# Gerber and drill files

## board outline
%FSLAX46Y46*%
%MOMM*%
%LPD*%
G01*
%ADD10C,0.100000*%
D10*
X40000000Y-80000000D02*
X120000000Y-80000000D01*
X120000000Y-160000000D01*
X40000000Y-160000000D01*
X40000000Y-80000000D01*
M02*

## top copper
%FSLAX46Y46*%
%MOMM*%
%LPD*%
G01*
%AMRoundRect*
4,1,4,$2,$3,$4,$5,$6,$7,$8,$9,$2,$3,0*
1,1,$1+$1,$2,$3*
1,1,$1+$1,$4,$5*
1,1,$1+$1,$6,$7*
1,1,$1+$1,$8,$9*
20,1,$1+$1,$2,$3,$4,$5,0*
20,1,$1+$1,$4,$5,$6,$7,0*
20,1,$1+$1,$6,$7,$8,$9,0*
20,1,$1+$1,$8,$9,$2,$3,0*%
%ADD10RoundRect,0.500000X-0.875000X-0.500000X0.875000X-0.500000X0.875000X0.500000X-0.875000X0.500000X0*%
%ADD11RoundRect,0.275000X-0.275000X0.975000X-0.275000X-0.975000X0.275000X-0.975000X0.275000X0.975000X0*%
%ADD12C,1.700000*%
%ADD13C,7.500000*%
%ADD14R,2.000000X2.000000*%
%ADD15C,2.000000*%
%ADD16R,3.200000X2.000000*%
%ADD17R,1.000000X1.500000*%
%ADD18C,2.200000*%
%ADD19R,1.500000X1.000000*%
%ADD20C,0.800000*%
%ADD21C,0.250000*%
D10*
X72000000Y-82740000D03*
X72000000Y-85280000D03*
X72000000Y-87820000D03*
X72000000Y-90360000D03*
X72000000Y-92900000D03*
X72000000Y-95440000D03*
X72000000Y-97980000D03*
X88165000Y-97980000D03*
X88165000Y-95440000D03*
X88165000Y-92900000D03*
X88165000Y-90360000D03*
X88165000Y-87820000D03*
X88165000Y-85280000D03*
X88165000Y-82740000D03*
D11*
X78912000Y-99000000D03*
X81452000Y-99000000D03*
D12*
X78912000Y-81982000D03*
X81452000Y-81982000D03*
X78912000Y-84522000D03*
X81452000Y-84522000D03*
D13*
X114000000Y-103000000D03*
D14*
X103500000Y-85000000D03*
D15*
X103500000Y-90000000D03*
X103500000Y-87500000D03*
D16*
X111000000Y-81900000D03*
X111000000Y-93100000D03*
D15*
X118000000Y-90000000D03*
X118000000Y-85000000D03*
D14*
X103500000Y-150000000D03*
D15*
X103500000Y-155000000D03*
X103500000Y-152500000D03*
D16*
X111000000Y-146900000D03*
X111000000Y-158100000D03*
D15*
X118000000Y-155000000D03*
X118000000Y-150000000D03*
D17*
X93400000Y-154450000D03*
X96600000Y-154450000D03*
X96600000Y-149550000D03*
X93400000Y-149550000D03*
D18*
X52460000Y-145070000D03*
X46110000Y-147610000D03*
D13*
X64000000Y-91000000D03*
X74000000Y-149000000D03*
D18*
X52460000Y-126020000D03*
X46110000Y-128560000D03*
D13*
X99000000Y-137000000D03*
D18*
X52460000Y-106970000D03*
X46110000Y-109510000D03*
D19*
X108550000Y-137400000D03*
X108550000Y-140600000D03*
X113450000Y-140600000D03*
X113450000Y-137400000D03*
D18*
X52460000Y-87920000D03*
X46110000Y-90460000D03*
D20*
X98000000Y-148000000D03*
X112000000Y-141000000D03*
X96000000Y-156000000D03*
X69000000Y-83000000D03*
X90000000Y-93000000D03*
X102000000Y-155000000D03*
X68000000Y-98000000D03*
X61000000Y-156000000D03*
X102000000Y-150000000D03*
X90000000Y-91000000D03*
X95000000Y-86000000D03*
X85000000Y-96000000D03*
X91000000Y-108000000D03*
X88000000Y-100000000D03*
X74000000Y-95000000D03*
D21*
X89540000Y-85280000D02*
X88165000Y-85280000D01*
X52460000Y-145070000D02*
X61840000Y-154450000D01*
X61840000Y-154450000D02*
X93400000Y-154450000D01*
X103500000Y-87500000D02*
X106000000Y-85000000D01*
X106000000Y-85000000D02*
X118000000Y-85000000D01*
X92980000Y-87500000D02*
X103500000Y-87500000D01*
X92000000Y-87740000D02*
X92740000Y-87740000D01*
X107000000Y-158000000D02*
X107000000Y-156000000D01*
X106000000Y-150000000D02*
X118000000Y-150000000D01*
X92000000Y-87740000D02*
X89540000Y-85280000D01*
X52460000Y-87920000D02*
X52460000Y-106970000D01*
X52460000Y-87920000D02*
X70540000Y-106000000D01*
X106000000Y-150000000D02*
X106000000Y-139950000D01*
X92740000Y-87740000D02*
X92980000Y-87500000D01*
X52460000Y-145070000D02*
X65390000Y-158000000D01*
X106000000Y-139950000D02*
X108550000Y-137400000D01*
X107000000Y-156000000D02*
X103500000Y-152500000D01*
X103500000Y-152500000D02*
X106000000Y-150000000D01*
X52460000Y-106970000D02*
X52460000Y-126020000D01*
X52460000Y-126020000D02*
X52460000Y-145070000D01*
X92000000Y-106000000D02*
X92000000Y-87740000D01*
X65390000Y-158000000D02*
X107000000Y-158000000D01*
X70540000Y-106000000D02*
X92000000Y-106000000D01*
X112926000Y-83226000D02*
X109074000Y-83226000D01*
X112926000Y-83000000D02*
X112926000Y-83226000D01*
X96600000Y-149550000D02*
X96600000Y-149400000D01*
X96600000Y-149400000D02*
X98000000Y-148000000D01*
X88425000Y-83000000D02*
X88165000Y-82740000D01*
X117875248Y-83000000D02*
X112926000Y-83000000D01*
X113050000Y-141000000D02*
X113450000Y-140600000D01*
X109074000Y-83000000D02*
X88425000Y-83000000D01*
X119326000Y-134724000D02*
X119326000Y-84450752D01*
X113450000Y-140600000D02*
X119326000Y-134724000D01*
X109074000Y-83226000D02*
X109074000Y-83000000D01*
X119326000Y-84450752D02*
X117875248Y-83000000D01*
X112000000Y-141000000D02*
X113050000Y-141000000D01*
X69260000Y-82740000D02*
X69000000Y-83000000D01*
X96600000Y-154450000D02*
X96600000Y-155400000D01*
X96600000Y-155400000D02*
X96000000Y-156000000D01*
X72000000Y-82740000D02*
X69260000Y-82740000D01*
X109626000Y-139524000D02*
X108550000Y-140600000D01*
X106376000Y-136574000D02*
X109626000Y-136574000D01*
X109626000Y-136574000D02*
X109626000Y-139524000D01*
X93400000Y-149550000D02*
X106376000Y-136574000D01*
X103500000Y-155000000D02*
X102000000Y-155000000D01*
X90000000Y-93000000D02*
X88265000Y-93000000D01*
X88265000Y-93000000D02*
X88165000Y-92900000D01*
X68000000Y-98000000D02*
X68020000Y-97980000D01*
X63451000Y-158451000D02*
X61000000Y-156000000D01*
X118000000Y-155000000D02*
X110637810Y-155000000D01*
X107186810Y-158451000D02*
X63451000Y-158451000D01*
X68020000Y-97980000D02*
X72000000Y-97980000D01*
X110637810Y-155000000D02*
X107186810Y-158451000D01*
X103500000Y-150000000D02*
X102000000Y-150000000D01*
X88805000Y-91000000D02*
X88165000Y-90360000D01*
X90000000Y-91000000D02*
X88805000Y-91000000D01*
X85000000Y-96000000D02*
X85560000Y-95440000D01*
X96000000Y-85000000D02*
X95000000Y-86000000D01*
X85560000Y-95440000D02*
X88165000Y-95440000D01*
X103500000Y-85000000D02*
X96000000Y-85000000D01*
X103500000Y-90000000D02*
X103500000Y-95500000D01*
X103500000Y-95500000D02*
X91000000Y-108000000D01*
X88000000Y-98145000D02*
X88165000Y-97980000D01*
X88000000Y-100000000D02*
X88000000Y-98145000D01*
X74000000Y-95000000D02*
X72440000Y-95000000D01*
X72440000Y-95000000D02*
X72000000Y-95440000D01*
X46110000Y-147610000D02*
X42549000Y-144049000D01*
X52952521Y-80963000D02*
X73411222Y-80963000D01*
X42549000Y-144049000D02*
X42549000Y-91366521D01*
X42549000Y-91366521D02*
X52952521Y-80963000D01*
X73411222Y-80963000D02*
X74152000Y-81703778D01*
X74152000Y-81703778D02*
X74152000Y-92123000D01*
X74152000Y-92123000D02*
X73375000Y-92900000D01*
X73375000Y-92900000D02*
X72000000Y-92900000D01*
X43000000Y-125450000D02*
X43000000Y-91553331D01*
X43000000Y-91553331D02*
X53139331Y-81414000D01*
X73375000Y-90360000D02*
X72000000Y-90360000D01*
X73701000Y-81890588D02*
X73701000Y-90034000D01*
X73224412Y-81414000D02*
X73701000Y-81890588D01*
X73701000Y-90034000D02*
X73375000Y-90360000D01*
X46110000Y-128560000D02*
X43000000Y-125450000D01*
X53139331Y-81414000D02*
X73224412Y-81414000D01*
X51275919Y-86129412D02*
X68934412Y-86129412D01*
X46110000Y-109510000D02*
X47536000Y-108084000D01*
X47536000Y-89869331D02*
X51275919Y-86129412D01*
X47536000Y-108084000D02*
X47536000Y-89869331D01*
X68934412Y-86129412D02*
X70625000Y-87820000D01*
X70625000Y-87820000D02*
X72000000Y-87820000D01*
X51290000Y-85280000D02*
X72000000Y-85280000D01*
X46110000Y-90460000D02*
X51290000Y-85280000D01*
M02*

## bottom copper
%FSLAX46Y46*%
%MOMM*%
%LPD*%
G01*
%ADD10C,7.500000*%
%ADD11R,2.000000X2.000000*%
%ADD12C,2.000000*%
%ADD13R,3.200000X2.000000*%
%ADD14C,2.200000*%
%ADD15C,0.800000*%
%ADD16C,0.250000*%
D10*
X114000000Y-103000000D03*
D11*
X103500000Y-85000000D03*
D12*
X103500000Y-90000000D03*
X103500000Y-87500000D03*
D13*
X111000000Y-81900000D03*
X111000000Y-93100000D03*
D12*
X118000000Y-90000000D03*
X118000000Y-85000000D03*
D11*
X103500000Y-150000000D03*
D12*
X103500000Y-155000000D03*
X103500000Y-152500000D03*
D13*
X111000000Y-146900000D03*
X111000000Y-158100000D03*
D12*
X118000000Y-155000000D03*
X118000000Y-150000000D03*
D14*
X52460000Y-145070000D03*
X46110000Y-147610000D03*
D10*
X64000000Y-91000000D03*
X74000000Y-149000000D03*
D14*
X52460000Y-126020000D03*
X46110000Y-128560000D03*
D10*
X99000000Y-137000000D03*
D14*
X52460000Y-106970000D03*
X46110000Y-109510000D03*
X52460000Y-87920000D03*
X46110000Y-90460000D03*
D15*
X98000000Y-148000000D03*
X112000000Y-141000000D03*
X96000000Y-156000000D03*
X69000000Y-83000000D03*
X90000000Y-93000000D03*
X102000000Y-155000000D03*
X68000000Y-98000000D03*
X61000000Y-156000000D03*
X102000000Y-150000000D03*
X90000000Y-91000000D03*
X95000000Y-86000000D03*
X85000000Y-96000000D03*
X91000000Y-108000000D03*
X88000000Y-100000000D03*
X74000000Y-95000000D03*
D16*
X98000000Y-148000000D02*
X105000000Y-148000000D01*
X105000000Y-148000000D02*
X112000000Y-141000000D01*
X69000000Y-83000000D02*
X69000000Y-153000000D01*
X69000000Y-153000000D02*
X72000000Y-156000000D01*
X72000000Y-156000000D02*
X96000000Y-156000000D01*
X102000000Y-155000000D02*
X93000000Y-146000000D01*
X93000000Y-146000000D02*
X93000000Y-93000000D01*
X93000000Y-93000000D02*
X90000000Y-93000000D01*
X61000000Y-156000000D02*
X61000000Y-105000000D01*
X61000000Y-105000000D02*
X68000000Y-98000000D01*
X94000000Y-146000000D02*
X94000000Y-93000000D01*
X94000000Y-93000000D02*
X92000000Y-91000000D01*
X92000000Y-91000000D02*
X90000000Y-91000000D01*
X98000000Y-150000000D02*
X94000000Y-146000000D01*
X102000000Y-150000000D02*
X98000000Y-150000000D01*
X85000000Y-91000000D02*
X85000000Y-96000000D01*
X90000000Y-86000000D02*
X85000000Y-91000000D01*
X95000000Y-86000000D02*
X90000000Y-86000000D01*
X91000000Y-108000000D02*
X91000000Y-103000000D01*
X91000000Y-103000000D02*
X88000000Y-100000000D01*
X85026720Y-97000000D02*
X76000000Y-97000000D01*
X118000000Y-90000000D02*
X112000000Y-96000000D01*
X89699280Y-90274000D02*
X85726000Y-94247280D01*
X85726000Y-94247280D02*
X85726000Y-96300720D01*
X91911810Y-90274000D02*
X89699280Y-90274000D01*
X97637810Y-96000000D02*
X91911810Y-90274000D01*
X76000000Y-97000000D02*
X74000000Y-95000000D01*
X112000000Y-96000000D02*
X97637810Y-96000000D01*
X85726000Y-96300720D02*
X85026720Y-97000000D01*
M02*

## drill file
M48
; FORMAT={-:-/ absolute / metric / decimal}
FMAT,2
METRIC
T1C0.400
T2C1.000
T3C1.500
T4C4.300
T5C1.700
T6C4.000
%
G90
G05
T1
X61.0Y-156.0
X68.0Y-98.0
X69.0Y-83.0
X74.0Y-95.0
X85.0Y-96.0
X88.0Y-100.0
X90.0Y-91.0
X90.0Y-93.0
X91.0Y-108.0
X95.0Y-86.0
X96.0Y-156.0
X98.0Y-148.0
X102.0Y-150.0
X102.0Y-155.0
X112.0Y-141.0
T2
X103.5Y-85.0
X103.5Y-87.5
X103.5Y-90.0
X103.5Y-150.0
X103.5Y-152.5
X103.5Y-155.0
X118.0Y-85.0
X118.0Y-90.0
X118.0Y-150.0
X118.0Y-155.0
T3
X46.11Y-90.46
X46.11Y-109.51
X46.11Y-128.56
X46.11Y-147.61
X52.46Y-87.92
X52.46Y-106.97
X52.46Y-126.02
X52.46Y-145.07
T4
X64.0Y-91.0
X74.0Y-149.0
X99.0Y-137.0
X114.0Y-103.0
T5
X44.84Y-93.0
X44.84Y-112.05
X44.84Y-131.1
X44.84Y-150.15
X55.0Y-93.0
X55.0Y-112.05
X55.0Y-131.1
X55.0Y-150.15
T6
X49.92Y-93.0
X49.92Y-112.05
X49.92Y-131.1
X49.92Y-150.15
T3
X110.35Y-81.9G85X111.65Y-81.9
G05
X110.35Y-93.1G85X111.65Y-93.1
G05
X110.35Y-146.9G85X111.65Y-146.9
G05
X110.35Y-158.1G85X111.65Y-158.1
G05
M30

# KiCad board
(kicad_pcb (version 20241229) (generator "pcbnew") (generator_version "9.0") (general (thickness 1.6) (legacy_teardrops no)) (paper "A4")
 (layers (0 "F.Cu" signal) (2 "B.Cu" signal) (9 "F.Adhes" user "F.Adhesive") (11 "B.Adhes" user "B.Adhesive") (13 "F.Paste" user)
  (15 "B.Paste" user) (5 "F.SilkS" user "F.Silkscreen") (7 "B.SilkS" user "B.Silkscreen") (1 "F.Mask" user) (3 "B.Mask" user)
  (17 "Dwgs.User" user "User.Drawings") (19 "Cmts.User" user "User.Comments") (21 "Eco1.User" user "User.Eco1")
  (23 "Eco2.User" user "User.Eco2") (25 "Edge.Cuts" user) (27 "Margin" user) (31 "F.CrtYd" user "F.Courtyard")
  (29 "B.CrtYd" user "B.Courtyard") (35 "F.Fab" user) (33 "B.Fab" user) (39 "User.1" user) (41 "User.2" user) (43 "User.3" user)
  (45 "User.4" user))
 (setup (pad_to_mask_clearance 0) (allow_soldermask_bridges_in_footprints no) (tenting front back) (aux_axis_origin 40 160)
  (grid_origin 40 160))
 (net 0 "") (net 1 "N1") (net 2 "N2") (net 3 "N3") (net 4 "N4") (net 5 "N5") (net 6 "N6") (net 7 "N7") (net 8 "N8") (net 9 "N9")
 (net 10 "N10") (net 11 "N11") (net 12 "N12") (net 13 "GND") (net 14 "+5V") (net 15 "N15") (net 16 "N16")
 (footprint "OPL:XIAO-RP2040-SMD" (layer "F.Cu") (at 80 90.36)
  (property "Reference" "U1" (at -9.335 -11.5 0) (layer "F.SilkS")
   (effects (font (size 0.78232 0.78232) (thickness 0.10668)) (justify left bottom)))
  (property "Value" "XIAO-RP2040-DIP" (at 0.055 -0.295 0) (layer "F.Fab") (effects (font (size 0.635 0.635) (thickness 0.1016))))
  (pad "1" smd roundrect (at -8 -7.62) (size 2.75 2) (layers "F.Cu" "F.Mask" "F.Paste") (roundrect_rratio 0.25) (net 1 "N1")
   (solder_mask_margin 0.0508) (thermal_bridge_angle 45))
  (pad "2" smd roundrect (at -8 -5.08) (size 2.75 2) (layers "F.Cu" "F.Mask" "F.Paste") (roundrect_rratio 0.25) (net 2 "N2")
   (solder_mask_margin 0.0508) (thermal_bridge_angle 45))
  (pad "3" smd roundrect (at -8 -2.54) (size 2.75 2) (layers "F.Cu" "F.Mask" "F.Paste") (roundrect_rratio 0.25) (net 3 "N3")
   (solder_mask_margin 0.0508) (thermal_bridge_angle 45))
  (pad "4" smd roundrect (at -8 0) (size 2.75 2) (layers "F.Cu" "F.Mask" "F.Paste") (roundrect_rratio 0.25) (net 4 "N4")
   (solder_mask_margin 0.0508) (thermal_bridge_angle 45))
  (pad "5" smd roundrect (at -8 2.54) (size 2.75 2) (layers "F.Cu" "F.Mask" "F.Paste") (roundrect_rratio 0.25) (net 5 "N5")
   (solder_mask_margin 0.0508) (thermal_bridge_angle 45))
  (pad "6" smd roundrect (at -8 5.08) (size 2.75 2) (layers "F.Cu" "F.Mask" "F.Paste") (roundrect_rratio 0.25) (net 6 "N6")
   (solder_mask_margin 0.0508) (thermal_bridge_angle 45))
  (pad "7" smd roundrect (at -8 7.62) (size 2.75 2) (layers "F.Cu" "F.Mask" "F.Paste") (roundrect_rratio 0.25) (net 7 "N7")
   (solder_mask_margin 0.0508) (thermal_bridge_angle 45))
  (pad "8" smd roundrect (at 8.165 7.62) (size 2.75 2) (layers "F.Cu" "F.Mask" "F.Paste") (roundrect_rratio 0.25) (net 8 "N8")
   (solder_mask_margin 0.0508) (thermal_bridge_angle 45))
  (pad "9" smd roundrect (at 8.165 5.08) (size 2.75 2) (layers "F.Cu" "F.Mask" "F.Paste") (roundrect_rratio 0.25) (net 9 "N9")
   (solder_mask_margin 0.0508) (thermal_bridge_angle 45))
  (pad "10" smd roundrect (at 8.165 2.54) (size 2.75 2) (layers "F.Cu" "F.Mask" "F.Paste") (roundrect_rratio 0.25) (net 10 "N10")
   (solder_mask_margin 0.0508) (thermal_bridge_angle 45))
  (pad "11" smd roundrect (at 8.165 0) (size 2.75 2) (layers "F.Cu" "F.Mask" "F.Paste") (roundrect_rratio 0.25) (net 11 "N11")
   (solder_mask_margin 0.0508) (thermal_bridge_angle 45))
  (pad "12" smd roundrect (at 8.165 -2.54) (size 2.75 2) (layers "F.Cu" "F.Mask" "F.Paste") (roundrect_rratio 0.25) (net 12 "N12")
   (solder_mask_margin 0.0508) (thermal_bridge_angle 45))
  (pad "13" smd roundrect (at 8.165 -5.08) (size 2.75 2) (layers "F.Cu" "F.Mask" "F.Paste") (roundrect_rratio 0.25) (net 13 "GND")
   (solder_mask_margin 0.0508) (thermal_bridge_angle 45))
  (pad "14" smd roundrect (at 8.165 -7.62) (size 2.75 2) (layers "F.Cu" "F.Mask" "F.Paste") (roundrect_rratio 0.25) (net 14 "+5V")
   (solder_mask_margin 0.0508) (thermal_bridge_angle 45))
  (pad "15" smd roundrect (at -1.088 8.64 270) (size 2.5 1.1) (layers "F.Cu" "F.Mask" "F.Paste") (roundrect_rratio 0.25)
   (thermal_bridge_angle 45))
  (pad "16" smd roundrect (at 1.452 8.64 270) (size 2.5 1.1) (layers "F.Cu" "F.Mask" "F.Paste") (roundrect_rratio 0.25)
   (thermal_bridge_angle 45))
  (pad "17" smd circle (at -1.088 -8.378) (size 1.7 1.7) (layers "F.Cu" "F.Mask" "F.Paste"))
  (pad "18" smd circle (at 1.452 -8.378) (size 1.7 1.7) (layers "F.Cu" "F.Mask" "F.Paste"))
  (pad "19" smd circle (at -1.088 -5.838) (size 1.7 1.7) (layers "F.Cu" "F.Mask" "F.Paste"))
  (pad "20" smd circle (at 1.452 -5.838) (size 1.7 1.7) (layers "F.Cu" "F.Mask" "F.Paste")))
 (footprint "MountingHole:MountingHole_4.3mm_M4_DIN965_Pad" (layer "F.Cu") (at 114 103)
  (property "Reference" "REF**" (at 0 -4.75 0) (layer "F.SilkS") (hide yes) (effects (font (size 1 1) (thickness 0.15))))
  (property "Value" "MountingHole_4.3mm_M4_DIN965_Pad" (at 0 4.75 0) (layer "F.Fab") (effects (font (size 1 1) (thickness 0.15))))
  (pad "1" thru_hole circle (at 0 0) (size 7.5 7.5) (drill 4.3) (layers "*.Cu" "*.Mask") (remove_unused_layers no)))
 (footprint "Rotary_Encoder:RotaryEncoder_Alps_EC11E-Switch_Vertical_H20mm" (layer "F.Cu") (at 103.5 85)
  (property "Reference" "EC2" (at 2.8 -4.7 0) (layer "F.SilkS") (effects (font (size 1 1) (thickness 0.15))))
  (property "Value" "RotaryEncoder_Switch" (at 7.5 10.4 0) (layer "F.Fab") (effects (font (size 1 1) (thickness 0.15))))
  (pad "A" thru_hole rect (at 0 0) (size 2 2) (drill 1) (layers "*.Cu" "*.Mask") (remove_unused_layers no) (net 9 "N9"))
  (pad "B" thru_hole circle (at 0 5) (size 2 2) (drill 1) (layers "*.Cu" "*.Mask") (remove_unused_layers no) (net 8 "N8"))
  (pad "C" thru_hole circle (at 0 2.5) (size 2 2) (drill 1) (layers "*.Cu" "*.Mask") (remove_unused_layers no) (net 13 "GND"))
  (pad "MP" thru_hole rect (at 7.5 -3.1) (size 3.2 2) (drill oval 2.8 1.5) (layers "*.Cu" "*.Mask") (remove_unused_layers no))
  (pad "MP" thru_hole rect (at 7.5 8.1) (size 3.2 2) (drill oval 2.8 1.5) (layers "*.Cu" "*.Mask") (remove_unused_layers no))
  (pad "S1" thru_hole circle (at 14.5 5) (size 2 2) (drill 1) (layers "*.Cu" "*.Mask") (remove_unused_layers no) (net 6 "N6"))
  (pad "S2" thru_hole circle (at 14.5 0) (size 2 2) (drill 1) (layers "*.Cu" "*.Mask") (remove_unused_layers no) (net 13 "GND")))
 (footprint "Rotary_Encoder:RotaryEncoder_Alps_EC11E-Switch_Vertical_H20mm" (layer "F.Cu") (at 103.5 150)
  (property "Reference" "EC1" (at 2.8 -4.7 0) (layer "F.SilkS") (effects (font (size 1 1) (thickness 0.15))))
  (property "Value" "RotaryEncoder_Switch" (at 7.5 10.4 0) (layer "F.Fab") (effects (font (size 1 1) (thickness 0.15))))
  (pad "A" thru_hole rect (at 0 0) (size 2 2) (drill 1) (layers "*.Cu" "*.Mask") (remove_unused_layers no) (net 11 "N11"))
  (pad "B" thru_hole circle (at 0 5) (size 2 2) (drill 1) (layers "*.Cu" "*.Mask") (remove_unused_layers no) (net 10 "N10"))
  (pad "C" thru_hole circle (at 0 2.5) (size 2 2) (drill 1) (layers "*.Cu" "*.Mask") (remove_unused_layers no) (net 13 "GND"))
  (pad "MP" thru_hole rect (at 7.5 -3.1) (size 3.2 2) (drill oval 2.8 1.5) (layers "*.Cu" "*.Mask") (remove_unused_layers no))
  (pad "MP" thru_hole rect (at 7.5 8.1) (size 3.2 2) (drill oval 2.8 1.5) (layers "*.Cu" "*.Mask") (remove_unused_layers no))
  (pad "S1" thru_hole circle (at 14.5 5) (size 2 2) (drill 1) (layers "*.Cu" "*.Mask") (remove_unused_layers no) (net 7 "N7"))
  (pad "S2" thru_hole circle (at 14.5 0) (size 2 2) (drill 1) (layers "*.Cu" "*.Mask") (remove_unused_layers no) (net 13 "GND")))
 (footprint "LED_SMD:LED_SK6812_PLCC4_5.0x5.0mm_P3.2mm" (layer "F.Cu") (at 95 152 90)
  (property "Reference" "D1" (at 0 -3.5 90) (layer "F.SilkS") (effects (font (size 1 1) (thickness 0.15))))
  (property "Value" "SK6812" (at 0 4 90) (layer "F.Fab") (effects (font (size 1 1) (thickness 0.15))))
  (pad "1" smd rect (at -2.45 -1.6 270) (size 1.5 1) (layers "F.Cu" "F.Mask" "F.Paste") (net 13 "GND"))
  (pad "2" smd rect (at -2.45 1.6 270) (size 1.5 1) (layers "F.Cu" "F.Mask" "F.Paste") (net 1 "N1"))
  (pad "3" smd rect (at 2.45 1.6 270) (size 1.5 1) (layers "F.Cu" "F.Mask" "F.Paste") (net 14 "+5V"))
  (pad "4" smd rect (at 2.45 -1.6 270) (size 1.5 1) (layers "F.Cu" "F.Mask" "F.Paste") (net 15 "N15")))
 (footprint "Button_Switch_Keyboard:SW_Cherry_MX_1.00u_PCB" (layer "F.Cu") (at 52.46 145.07)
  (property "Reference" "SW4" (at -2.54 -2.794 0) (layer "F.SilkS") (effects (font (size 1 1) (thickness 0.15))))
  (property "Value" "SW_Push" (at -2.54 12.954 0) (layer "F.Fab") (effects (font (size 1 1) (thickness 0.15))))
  (pad "" np_thru_hole circle (at -7.62 5.08) (size 1.7 1.7) (drill 1.7) (layers "*.Cu" "*.Mask"))
  (pad "" np_thru_hole circle (at -2.54 5.08) (size 4 4) (drill 4) (layers "*.Cu" "*.Mask"))
  (pad "" np_thru_hole circle (at 2.54 5.08) (size 1.7 1.7) (drill 1.7) (layers "*.Cu" "*.Mask"))
  (pad "1" thru_hole circle (at 0 0) (size 2.2 2.2) (drill 1.5) (layers "*.Cu" "*.Mask") (remove_unused_layers no) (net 13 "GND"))
  (pad "2" thru_hole circle (at -6.35 2.54) (size 2.2 2.2) (drill 1.5) (layers "*.Cu" "*.Mask") (remove_unused_layers no) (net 5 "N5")))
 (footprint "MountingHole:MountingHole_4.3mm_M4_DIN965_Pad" (layer "F.Cu") (at 64 91)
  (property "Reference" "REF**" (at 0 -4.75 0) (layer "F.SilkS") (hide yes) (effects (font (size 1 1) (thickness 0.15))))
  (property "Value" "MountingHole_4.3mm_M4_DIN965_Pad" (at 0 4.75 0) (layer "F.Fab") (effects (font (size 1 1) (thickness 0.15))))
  (pad "1" thru_hole circle (at 0 0) (size 7.5 7.5) (drill 4.3) (layers "*.Cu" "*.Mask") (remove_unused_layers no)))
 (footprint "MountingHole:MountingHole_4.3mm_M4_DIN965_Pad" (layer "F.Cu") (at 74 149)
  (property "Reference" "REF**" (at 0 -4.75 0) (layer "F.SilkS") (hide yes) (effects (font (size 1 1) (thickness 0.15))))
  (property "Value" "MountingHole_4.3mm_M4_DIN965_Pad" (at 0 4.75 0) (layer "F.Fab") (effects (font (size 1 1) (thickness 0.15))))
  (pad "1" thru_hole circle (at 0 0) (size 7.5 7.5) (drill 4.3) (layers "*.Cu" "*.Mask") (remove_unused_layers no)))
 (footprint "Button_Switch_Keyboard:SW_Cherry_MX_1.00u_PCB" (layer "F.Cu") (at 52.46 126.02)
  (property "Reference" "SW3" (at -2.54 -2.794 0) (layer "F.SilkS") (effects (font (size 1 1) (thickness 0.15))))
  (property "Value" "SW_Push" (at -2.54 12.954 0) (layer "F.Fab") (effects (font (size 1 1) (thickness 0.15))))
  (pad "" np_thru_hole circle (at -7.62 5.08) (size 1.7 1.7) (drill 1.7) (layers "*.Cu" "*.Mask"))
  (pad "" np_thru_hole circle (at -2.54 5.08) (size 4 4) (drill 4) (layers "*.Cu" "*.Mask"))
  (pad "" np_thru_hole circle (at 2.54 5.08) (size 1.7 1.7) (drill 1.7) (layers "*.Cu" "*.Mask"))
  (pad "1" thru_hole circle (at 0 0) (size 2.2 2.2) (drill 1.5) (layers "*.Cu" "*.Mask") (remove_unused_layers no) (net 13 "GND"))
  (pad "2" thru_hole circle (at -6.35 2.54) (size 2.2 2.2) (drill 1.5) (layers "*.Cu" "*.Mask") (remove_unused_layers no) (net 4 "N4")))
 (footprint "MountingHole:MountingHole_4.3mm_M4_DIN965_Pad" (layer "F.Cu") (at 99 137)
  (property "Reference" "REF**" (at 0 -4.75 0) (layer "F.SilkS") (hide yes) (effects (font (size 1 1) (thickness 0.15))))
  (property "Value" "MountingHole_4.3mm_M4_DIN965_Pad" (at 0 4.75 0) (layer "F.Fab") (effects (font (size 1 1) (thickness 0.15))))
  (pad "1" thru_hole circle (at 0 0) (size 7.5 7.5) (drill 4.3) (layers "*.Cu" "*.Mask") (remove_unused_layers no)))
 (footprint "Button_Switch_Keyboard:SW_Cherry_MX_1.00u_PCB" (layer "F.Cu") (at 52.46 106.97)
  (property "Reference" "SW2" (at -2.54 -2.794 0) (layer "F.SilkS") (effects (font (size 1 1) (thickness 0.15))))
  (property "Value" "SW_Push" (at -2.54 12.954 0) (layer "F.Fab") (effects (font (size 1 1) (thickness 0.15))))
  (pad "" np_thru_hole circle (at -7.62 5.08) (size 1.7 1.7) (drill 1.7) (layers "*.Cu" "*.Mask"))
  (pad "" np_thru_hole circle (at -2.54 5.08) (size 4 4) (drill 4) (layers "*.Cu" "*.Mask"))
  (pad "" np_thru_hole circle (at 2.54 5.08) (size 1.7 1.7) (drill 1.7) (layers "*.Cu" "*.Mask"))
  (pad "1" thru_hole circle (at 0 0) (size 2.2 2.2) (drill 1.5) (layers "*.Cu" "*.Mask") (remove_unused_layers no) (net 13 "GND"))
  (pad "2" thru_hole circle (at -6.35 2.54) (size 2.2 2.2) (drill 1.5) (layers "*.Cu" "*.Mask") (remove_unused_layers no) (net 3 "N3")))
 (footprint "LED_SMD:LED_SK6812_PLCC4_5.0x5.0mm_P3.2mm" (layer "F.Cu") (at 111 139)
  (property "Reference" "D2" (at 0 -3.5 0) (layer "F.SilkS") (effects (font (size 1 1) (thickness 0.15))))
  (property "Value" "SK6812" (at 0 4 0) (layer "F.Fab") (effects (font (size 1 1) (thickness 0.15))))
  (pad "1" smd rect (at -2.45 -1.6 180) (size 1.5 1) (layers "F.Cu" "F.Mask" "F.Paste") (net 13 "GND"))
  (pad "2" smd rect (at -2.45 1.6 180) (size 1.5 1) (layers "F.Cu" "F.Mask" "F.Paste") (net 15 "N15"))
  (pad "3" smd rect (at 2.45 1.6 180) (size 1.5 1) (layers "F.Cu" "F.Mask" "F.Paste") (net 14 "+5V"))
  (pad "4" smd rect (at 2.45 -1.6 180) (size 1.5 1) (layers "F.Cu" "F.Mask" "F.Paste") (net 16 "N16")))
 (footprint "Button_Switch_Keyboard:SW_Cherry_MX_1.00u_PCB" (layer "F.Cu") (at 52.46 87.92)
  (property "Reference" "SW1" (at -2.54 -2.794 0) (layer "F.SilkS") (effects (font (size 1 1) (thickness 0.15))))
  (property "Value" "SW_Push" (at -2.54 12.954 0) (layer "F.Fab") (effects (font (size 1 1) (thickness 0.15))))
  (pad "" np_thru_hole circle (at -7.62 5.08) (size 1.7 1.7) (drill 1.7) (layers "*.Cu" "*.Mask"))
  (pad "" np_thru_hole circle (at -2.54 5.08) (size 4 4) (drill 4) (layers "*.Cu" "*.Mask"))
  (pad "" np_thru_hole circle (at 2.54 5.08) (size 1.7 1.7) (drill 1.7) (layers "*.Cu" "*.Mask"))
  (pad "1" thru_hole circle (at 0 0) (size 2.2 2.2) (drill 1.5) (layers "*.Cu" "*.Mask") (remove_unused_layers no) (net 13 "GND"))
  (pad "2" thru_hole circle (at -6.35 2.54) (size 2.2 2.2) (drill 1.5) (layers "*.Cu" "*.Mask") (remove_unused_layers no) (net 2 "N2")))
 (gr_rect (start 40 80) (end 120 160) (stroke (width 0.1) (type solid)) (fill no) (layer "Edge.Cuts"))
 (segment (start 89.54 85.28) (end 88.165 85.28) (width 0.25) (layer "F.Cu") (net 13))
 (segment (start 52.46 145.07) (end 61.84 154.45) (width 0.25) (layer "F.Cu") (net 13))
 (segment (start 61.84 154.45) (end 93.4 154.45) (width 0.25) (layer "F.Cu") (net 13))
 (segment (start 103.5 87.5) (end 106 85) (width 0.25) (layer "F.Cu") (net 13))
 (segment (start 106 85) (end 118 85) (width 0.25) (layer "F.Cu") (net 13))
 (segment (start 92.98 87.5) (end 103.5 87.5) (width 0.25) (layer "F.Cu") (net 13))
 (segment (start 92 87.74) (end 92.74 87.74) (width 0.25) (layer "F.Cu") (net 13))
 (segment (start 107 158) (end 107 156) (width 0.25) (layer "F.Cu") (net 13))
 (segment (start 106 150) (end 118 150) (width 0.25) (layer "F.Cu") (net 13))
 (segment (start 92 87.74) (end 89.54 85.28) (width 0.25) (layer "F.Cu") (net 13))
 (segment (start 52.46 87.92) (end 52.46 106.97) (width 0.25) (layer "F.Cu") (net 13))
 (segment (start 52.46 87.92) (end 70.54 106) (width 0.25) (layer "F.Cu") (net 13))
 (segment (start 106 150) (end 106 139.95) (width 0.25) (layer "F.Cu") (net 13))
 (segment (start 92.74 87.74) (end 92.98 87.5) (width 0.25) (layer "F.Cu") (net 13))
 (segment (start 52.46 145.07) (end 65.39 158) (width 0.25) (layer "F.Cu") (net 13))
 (segment (start 106 139.95) (end 108.55 137.4) (width 0.25) (layer "F.Cu") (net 13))
 (segment (start 107 156) (end 103.5 152.5) (width 0.25) (layer "F.Cu") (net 13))
 (segment (start 103.5 152.5) (end 106 150) (width 0.25) (layer "F.Cu") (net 13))
 (segment (start 52.46 106.97) (end 52.46 126.02) (width 0.25) (layer "F.Cu") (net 13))
 (segment (start 52.46 126.02) (end 52.46 145.07) (width 0.25) (layer "F.Cu") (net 13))
 (segment (start 92 106) (end 92 87.74) (width 0.25) (layer "F.Cu") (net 13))
 (segment (start 65.39 158) (end 107 158) (width 0.25) (layer "F.Cu") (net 13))
 (segment (start 70.54 106) (end 92 106) (width 0.25) (layer "F.Cu") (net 13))
 (segment (start 112.926 83.226) (end 109.074 83.226) (width 0.25) (layer "F.Cu") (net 14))
 (segment (start 112.926 83) (end 112.926 83.226) (width 0.25) (layer "F.Cu") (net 14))
 (segment (start 96.6 149.55) (end 96.6 149.4) (width 0.25) (layer "F.Cu") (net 14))
 (segment (start 96.6 149.4) (end 98 148) (width 0.25) (layer "F.Cu") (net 14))
 (segment (start 88.425 83) (end 88.165 82.74) (width 0.25) (layer "F.Cu") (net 14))
 (segment (start 117.875248 83) (end 112.926 83) (width 0.25) (layer "F.Cu") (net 14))
 (segment (start 113.05 141) (end 113.45 140.6) (width 0.25) (layer "F.Cu") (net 14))
 (segment (start 109.074 83) (end 88.425 83) (width 0.25) (layer "F.Cu") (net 14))
 (segment (start 119.326 134.724) (end 119.326 84.450752) (width 0.25) (layer "F.Cu") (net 14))
 (segment (start 113.45 140.6) (end 119.326 134.724) (width 0.25) (layer "F.Cu") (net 14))
 (segment (start 109.074 83.226) (end 109.074 83) (width 0.25) (layer "F.Cu") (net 14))
 (segment (start 119.326 84.450752) (end 117.875248 83) (width 0.25) (layer "F.Cu") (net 14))
 (segment (start 112 141) (end 113.05 141) (width 0.25) (layer "F.Cu") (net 14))
 (via (at 98 148) (size 0.8) (drill 0.4) (layers "F.Cu" "B.Cu") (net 14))
 (via (at 112 141) (size 0.8) (drill 0.4) (layers "F.Cu" "B.Cu") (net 14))
 (segment (start 98 148) (end 105 148) (width 0.25) (layer "B.Cu") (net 14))
 (segment (start 105 148) (end 112 141) (width 0.25) (layer "B.Cu") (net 14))
 (segment (start 69.26 82.74) (end 69 83) (width 0.25) (layer "F.Cu") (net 1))
 (segment (start 96.6 154.45) (end 96.6 155.4) (width 0.25) (layer "F.Cu") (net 1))
 (segment (start 96.6 155.4) (end 96 156) (width 0.25) (layer "F.Cu") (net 1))
 (segment (start 72 82.74) (end 69.26 82.74) (width 0.25) (layer "F.Cu") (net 1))
 (via (at 96 156) (size 0.8) (drill 0.4) (layers "F.Cu" "B.Cu") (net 1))
 (via (at 69 83) (size 0.8) (drill 0.4) (layers "F.Cu" "B.Cu") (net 1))
 (segment (start 69 83) (end 69 153) (width 0.25) (layer "B.Cu") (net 1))
 (segment (start 69 153) (end 72 156) (width 0.25) (layer "B.Cu") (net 1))
 (segment (start 72 156) (end 96 156) (width 0.25) (layer "B.Cu") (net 1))
 (segment (start 109.626 139.524) (end 108.55 140.6) (width 0.25) (layer "F.Cu") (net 15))
 (segment (start 106.376 136.574) (end 109.626 136.574) (width 0.25) (layer "F.Cu") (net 15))
 (segment (start 109.626 136.574) (end 109.626 139.524) (width 0.25) (layer "F.Cu") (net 15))
 (segment (start 93.4 149.55) (end 106.376 136.574) (width 0.25) (layer "F.Cu") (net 15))
 (segment (start 103.5 155) (end 102 155) (width 0.25) (layer "F.Cu") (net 10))
 (segment (start 90 93) (end 88.265 93) (width 0.25) (layer "F.Cu") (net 10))
 (segment (start 88.265 93) (end 88.165 92.9) (width 0.25) (layer "F.Cu") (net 10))
 (via (at 90 93) (size 0.8) (drill 0.4) (layers "F.Cu" "B.Cu") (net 10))
 (via (at 102 155) (size 0.8) (drill 0.4) (layers "F.Cu" "B.Cu") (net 10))
 (segment (start 102 155) (end 93 146) (width 0.25) (layer "B.Cu") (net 10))
 (segment (start 93 146) (end 93 93) (width 0.25) (layer "B.Cu") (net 10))
 (segment (start 93 93) (end 90 93) (width 0.25) (layer "B.Cu") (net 10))
 (segment (start 68 98) (end 68.02 97.98) (width 0.25) (layer "F.Cu") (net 7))
 (segment (start 63.451 158.451) (end 61 156) (width 0.25) (layer "F.Cu") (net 7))
 (segment (start 118 155) (end 110.63781 155) (width 0.25) (layer "F.Cu") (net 7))
 (segment (start 107.18681 158.451) (end 63.451 158.451) (width 0.25) (layer "F.Cu") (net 7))
 (segment (start 68.02 97.98) (end 72 97.98) (width 0.25) (layer "F.Cu") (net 7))
 (segment (start 110.63781 155) (end 107.18681 158.451) (width 0.25) (layer "F.Cu") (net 7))
 (via (at 68 98) (size 0.8) (drill 0.4) (layers "F.Cu" "B.Cu") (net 7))
 (via (at 61 156) (size 0.8) (drill 0.4) (layers "F.Cu" "B.Cu") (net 7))
 (segment (start 61 156) (end 61 105) (width 0.25) (layer "B.Cu") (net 7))
 (segment (start 61 105) (end 68 98) (width 0.25) (layer "B.Cu") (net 7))
 (segment (start 103.5 150) (end 102 150) (width 0.25) (layer "F.Cu") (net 11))
 (segment (start 88.805 91) (end 88.165 90.36) (width 0.25) (layer "F.Cu") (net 11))
 (segment (start 90 91) (end 88.805 91) (width 0.25) (layer "F.Cu") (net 11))
 (via (at 102 150) (size 0.8) (drill 0.4) (layers "F.Cu" "B.Cu") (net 11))
 (via (at 90 91) (size 0.8) (drill 0.4) (layers "F.Cu" "B.Cu") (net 11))
 (segment (start 94 146) (end 94 93) (width 0.25) (layer "B.Cu") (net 11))
 (segment (start 94 93) (end 92 91) (width 0.25) (layer "B.Cu") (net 11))
 (segment (start 92 91) (end 90 91) (width 0.25) (layer "B.Cu") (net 11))
 (segment (start 98 150) (end 94 146) (width 0.25) (layer "B.Cu") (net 11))
 (segment (start 102 150) (end 98 150) (width 0.25) (layer "B.Cu") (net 11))
 (segment (start 85 96) (end 85.56 95.44) (width 0.25) (layer "F.Cu") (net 9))
 (segment (start 96 85) (end 95 86) (width 0.25) (layer "F.Cu") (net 9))
 (segment (start 85.56 95.44) (end 88.165 95.44) (width 0.25) (layer "F.Cu") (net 9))
 (segment (start 103.5 85) (end 96 85) (width 0.25) (layer "F.Cu") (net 9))
 (via (at 95 86) (size 0.8) (drill 0.4) (layers "F.Cu" "B.Cu") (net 9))
 (via (at 85 96) (size 0.8) (drill 0.4) (layers "F.Cu" "B.Cu") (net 9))
 (segment (start 85 91) (end 85 96) (width 0.25) (layer "B.Cu") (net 9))
 (segment (start 90 86) (end 85 91) (width 0.25) (layer "B.Cu") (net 9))
 (segment (start 95 86) (end 90 86) (width 0.25) (layer "B.Cu") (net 9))
 (segment (start 103.5 90) (end 103.5 95.5) (width 0.25) (layer "F.Cu") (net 8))
 (segment (start 103.5 95.5) (end 91 108) (width 0.25) (layer "F.Cu") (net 8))
 (segment (start 88 98.145) (end 88.165 97.98) (width 0.25) (layer "F.Cu") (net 8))
 (segment (start 88 100) (end 88 98.145) (width 0.25) (layer "F.Cu") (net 8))
 (via (at 91 108) (size 0.8) (drill 0.4) (layers "F.Cu" "B.Cu") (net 8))
 (via (at 88 100) (size 0.8) (drill 0.4) (layers "F.Cu" "B.Cu") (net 8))
 (segment (start 91 108) (end 91 103) (width 0.25) (layer "B.Cu") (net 8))
 (segment (start 91 103) (end 88 100) (width 0.25) (layer "B.Cu") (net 8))
 (segment (start 74 95) (end 72.44 95) (width 0.25) (layer "F.Cu") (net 6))
 (segment (start 72.44 95) (end 72 95.44) (width 0.25) (layer "F.Cu") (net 6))
 (via (at 74 95) (size 0.8) (drill 0.4) (layers "F.Cu" "B.Cu") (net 6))
 (segment (start 85.02672 97) (end 76 97) (width 0.25) (layer "B.Cu") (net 6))
 (segment (start 118 90) (end 112 96) (width 0.25) (layer "B.Cu") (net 6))
 (segment (start 89.69928 90.274) (end 85.726 94.24728) (width 0.25) (layer "B.Cu") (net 6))
 (segment (start 85.726 94.24728) (end 85.726 96.30072) (width 0.25) (layer "B.Cu") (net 6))
 (segment (start 91.91181 90.274) (end 89.69928 90.274) (width 0.25) (layer "B.Cu") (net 6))
 (segment (start 97.63781 96) (end 91.91181 90.274) (width 0.25) (layer "B.Cu") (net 6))
 (segment (start 76 97) (end 74 95) (width 0.25) (layer "B.Cu") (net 6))
 (segment (start 112 96) (end 97.63781 96) (width 0.25) (layer "B.Cu") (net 6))
 (segment (start 85.726 96.30072) (end 85.02672 97) (width 0.25) (layer "B.Cu") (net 6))
 (segment (start 46.11 147.61) (end 42.549 144.049) (width 0.25) (layer "F.Cu") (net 5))
 (segment (start 52.952521 80.963) (end 73.411222 80.963) (width 0.25) (layer "F.Cu") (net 5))
 (segment (start 42.549 144.049) (end 42.549 91.366521) (width 0.25) (layer "F.Cu") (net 5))
 (segment (start 42.549 91.366521) (end 52.952521 80.963) (width 0.25) (layer "F.Cu") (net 5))
 (segment (start 73.411222 80.963) (end 74.152 81.703778) (width 0.25) (layer "F.Cu") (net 5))
 (segment (start 74.152 81.703778) (end 74.152 92.123) (width 0.25) (layer "F.Cu") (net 5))
 (segment (start 74.152 92.123) (end 73.375 92.9) (width 0.25) (layer "F.Cu") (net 5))
 (segment (start 73.375 92.9) (end 72 92.9) (width 0.25) (layer "F.Cu") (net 5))
 (segment (start 43 125.45) (end 43 91.553331) (width 0.25) (layer "F.Cu") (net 4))
 (segment (start 43 91.553331) (end 53.139331 81.414) (width 0.25) (layer "F.Cu") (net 4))
 (segment (start 73.375 90.36) (end 72 90.36) (width 0.25) (layer "F.Cu") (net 4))
 (segment (start 73.701 81.890588) (end 73.701 90.034) (width 0.25) (layer "F.Cu") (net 4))
 (segment (start 73.224412 81.414) (end 73.701 81.890588) (width 0.25) (layer "F.Cu") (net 4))
 (segment (start 73.701 90.034) (end 73.375 90.36) (width 0.25) (layer "F.Cu") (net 4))
 (segment (start 46.11 128.56) (end 43 125.45) (width 0.25) (layer "F.Cu") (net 4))
 (segment (start 53.139331 81.414) (end 73.224412 81.414) (width 0.25) (layer "F.Cu") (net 4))
 (segment (start 51.275919 86.129412) (end 68.934412 86.129412) (width 0.25) (layer "F.Cu") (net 3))
 (segment (start 46.11 109.51) (end 47.536 108.084) (width 0.25) (layer "F.Cu") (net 3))
 (segment (start 47.536 89.869331) (end 51.275919 86.129412) (width 0.25) (layer "F.Cu") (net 3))
 (segment (start 47.536 108.084) (end 47.536 89.869331) (width 0.25) (layer "F.Cu") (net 3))
 (segment (start 68.934412 86.129412) (end 70.625 87.82) (width 0.25) (layer "F.Cu") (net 3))
 (segment (start 70.625 87.82) (end 72 87.82) (width 0.25) (layer "F.Cu") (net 3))
 (segment (start 51.29 85.28) (end 72 85.28) (width 0.25) (layer "F.Cu") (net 2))
 (segment (start 46.11 90.46) (end 51.29 85.28) (width 0.25) (layer "F.Cu") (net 2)))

